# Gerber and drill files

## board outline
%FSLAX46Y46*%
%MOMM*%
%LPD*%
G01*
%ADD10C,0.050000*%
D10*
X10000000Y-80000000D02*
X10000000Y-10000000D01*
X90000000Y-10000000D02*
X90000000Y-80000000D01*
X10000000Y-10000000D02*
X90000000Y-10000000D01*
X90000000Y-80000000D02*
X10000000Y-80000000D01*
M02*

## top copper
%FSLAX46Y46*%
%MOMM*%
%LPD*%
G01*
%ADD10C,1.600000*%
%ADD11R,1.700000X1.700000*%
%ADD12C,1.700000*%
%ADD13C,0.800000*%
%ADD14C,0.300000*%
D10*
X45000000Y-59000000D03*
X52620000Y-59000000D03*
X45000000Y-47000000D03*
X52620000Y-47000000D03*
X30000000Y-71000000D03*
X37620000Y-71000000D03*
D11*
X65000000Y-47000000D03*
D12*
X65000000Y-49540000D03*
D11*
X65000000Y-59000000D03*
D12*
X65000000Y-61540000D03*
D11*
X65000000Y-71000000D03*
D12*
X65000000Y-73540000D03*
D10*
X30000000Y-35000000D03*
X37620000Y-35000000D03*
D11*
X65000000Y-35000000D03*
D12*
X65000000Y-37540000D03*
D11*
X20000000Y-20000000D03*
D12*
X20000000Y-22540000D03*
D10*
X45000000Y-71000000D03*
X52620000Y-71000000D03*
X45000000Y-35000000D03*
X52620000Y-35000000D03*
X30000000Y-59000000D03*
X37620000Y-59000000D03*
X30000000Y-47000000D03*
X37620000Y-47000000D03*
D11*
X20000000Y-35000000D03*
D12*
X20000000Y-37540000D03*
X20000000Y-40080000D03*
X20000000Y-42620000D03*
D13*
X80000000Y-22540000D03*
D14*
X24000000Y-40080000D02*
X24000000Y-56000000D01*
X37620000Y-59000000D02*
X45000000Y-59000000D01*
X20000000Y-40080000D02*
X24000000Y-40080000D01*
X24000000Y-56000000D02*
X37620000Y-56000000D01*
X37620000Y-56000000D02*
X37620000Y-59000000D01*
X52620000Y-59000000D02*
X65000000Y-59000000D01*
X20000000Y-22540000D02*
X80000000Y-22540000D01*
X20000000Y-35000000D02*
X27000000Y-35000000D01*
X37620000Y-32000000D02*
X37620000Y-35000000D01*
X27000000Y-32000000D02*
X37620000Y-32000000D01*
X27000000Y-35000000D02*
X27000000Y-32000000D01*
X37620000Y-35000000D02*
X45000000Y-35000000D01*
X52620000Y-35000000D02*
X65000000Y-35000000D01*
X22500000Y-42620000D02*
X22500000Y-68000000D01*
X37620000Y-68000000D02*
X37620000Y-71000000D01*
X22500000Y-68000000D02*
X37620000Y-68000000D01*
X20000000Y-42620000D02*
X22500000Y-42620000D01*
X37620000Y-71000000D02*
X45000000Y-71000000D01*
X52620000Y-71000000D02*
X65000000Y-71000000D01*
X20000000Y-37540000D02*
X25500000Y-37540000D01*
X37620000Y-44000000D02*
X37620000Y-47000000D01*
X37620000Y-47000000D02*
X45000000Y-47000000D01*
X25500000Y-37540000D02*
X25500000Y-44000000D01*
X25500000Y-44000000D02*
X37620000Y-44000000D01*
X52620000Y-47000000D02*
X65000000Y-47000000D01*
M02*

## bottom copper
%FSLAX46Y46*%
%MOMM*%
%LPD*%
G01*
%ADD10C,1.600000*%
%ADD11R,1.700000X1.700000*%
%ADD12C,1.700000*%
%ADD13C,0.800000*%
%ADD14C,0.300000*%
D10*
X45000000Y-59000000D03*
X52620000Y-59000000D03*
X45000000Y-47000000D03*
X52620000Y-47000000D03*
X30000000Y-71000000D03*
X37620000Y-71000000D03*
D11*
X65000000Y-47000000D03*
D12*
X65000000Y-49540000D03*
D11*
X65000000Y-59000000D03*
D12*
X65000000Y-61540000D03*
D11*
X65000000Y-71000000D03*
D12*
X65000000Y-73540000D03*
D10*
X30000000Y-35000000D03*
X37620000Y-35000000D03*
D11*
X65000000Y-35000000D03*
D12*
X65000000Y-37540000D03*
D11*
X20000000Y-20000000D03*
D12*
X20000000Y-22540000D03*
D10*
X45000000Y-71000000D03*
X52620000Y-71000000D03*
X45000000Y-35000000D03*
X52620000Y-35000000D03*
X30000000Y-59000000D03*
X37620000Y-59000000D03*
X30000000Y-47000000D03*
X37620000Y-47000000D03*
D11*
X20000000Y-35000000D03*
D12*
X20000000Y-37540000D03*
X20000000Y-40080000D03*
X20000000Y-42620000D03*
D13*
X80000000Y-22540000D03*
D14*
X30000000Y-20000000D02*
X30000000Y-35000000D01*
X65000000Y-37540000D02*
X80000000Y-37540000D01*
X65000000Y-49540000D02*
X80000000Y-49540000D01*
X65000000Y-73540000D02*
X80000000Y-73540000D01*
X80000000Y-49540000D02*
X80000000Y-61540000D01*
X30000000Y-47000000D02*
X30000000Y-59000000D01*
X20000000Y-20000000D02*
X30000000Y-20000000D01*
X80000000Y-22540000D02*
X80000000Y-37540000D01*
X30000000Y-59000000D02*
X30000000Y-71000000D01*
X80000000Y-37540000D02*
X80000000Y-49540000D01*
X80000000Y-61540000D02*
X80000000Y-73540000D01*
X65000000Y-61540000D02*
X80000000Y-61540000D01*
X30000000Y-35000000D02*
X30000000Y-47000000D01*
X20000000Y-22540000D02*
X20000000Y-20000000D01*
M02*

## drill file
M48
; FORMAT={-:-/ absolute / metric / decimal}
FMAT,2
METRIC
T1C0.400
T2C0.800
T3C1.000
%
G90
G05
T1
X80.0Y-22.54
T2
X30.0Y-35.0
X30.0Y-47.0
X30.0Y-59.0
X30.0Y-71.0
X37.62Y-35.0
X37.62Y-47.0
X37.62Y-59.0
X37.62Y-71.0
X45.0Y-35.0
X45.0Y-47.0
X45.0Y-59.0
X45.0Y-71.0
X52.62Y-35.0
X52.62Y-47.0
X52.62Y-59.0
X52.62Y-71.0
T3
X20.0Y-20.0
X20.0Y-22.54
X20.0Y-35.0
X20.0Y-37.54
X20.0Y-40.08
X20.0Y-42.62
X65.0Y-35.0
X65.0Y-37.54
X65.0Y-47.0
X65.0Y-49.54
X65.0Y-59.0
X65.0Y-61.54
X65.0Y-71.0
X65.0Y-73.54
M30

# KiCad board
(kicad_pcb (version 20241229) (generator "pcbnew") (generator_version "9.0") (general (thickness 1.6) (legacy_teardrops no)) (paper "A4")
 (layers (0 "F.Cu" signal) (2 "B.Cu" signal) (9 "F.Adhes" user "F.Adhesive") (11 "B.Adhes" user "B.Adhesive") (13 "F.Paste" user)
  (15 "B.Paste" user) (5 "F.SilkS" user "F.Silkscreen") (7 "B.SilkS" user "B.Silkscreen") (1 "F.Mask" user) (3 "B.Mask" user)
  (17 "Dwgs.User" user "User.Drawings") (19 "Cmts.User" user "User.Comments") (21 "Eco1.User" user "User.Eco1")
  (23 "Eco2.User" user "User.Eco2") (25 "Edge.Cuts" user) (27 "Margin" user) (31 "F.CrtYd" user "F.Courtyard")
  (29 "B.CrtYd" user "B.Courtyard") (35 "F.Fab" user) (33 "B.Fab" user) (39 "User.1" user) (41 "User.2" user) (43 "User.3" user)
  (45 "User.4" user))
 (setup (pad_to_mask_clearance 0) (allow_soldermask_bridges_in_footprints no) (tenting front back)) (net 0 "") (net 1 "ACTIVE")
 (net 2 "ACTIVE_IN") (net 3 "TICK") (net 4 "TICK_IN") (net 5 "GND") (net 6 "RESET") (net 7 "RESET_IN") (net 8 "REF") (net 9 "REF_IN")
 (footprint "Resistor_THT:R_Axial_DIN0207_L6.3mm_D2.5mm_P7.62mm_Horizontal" (layer "F.Cu") (at 45 59)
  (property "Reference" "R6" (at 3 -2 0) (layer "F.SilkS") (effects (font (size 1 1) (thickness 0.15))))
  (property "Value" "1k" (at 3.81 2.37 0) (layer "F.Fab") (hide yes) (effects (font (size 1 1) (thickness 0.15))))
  (pad "1" thru_hole circle (at 0 0) (size 1.6 1.6) (drill 0.8) (layers "*.Cu" "*.Mask") (remove_unused_layers no) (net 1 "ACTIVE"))
  (pad "2" thru_hole circle (at 7.62 0) (size 1.6 1.6) (drill 0.8) (layers "*.Cu" "*.Mask") (remove_unused_layers no) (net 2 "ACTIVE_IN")))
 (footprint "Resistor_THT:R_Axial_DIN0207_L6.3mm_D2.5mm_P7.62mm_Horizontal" (layer "F.Cu") (at 45 47)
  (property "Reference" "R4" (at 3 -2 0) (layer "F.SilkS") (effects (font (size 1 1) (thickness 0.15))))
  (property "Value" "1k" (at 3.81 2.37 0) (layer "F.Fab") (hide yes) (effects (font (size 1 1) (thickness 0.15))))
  (pad "1" thru_hole circle (at 0 0) (size 1.6 1.6) (drill 0.8) (layers "*.Cu" "*.Mask") (remove_unused_layers no) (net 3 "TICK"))
  (pad "2" thru_hole circle (at 7.62 0) (size 1.6 1.6) (drill 0.8) (layers "*.Cu" "*.Mask") (remove_unused_layers no) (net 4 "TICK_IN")))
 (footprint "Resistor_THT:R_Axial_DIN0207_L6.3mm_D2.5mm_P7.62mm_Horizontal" (layer "F.Cu") (at 30 71)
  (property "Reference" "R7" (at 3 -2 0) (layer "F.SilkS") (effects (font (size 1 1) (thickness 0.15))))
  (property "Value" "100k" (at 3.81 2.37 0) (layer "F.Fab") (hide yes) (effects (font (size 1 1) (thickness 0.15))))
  (pad "1" thru_hole circle (at 0 0) (size 1.6 1.6) (drill 0.8) (layers "*.Cu" "*.Mask") (remove_unused_layers no) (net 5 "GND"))
  (pad "2" thru_hole circle (at 7.62 0) (size 1.6 1.6) (drill 0.8) (layers "*.Cu" "*.Mask") (remove_unused_layers no) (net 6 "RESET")))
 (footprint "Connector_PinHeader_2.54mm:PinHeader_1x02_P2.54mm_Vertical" (layer "F.Cu") (at 65 47)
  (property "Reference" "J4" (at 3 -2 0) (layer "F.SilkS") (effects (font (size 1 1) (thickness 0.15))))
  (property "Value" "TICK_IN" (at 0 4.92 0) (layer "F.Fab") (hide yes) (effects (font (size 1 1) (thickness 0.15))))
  (pad "1" thru_hole rect (at 0 0) (size 1.7 1.7) (drill 1) (layers "*.Cu" "*.Mask") (remove_unused_layers no) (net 4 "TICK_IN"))
  (pad "2" thru_hole circle (at 0 2.54) (size 1.7 1.7) (drill 1) (layers "*.Cu" "*.Mask") (remove_unused_layers no) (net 5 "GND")))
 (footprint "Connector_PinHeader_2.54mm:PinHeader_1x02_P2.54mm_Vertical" (layer "F.Cu") (at 65 59)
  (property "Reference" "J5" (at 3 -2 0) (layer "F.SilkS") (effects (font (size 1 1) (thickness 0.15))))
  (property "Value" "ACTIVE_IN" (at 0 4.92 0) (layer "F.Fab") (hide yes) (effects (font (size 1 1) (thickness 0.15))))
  (pad "1" thru_hole rect (at 0 0) (size 1.7 1.7) (drill 1) (layers "*.Cu" "*.Mask") (remove_unused_layers no) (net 2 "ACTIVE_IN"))
  (pad "2" thru_hole circle (at 0 2.54) (size 1.7 1.7) (drill 1) (layers "*.Cu" "*.Mask") (remove_unused_layers no) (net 5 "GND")))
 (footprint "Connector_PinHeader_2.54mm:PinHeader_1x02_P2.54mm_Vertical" (layer "F.Cu") (at 65 71)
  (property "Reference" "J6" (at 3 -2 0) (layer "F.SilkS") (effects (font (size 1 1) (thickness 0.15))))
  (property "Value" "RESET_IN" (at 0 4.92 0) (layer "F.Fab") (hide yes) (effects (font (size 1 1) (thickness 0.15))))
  (pad "1" thru_hole rect (at 0 0) (size 1.7 1.7) (drill 1) (layers "*.Cu" "*.Mask") (remove_unused_layers no) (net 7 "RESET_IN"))
  (pad "2" thru_hole circle (at 0 2.54) (size 1.7 1.7) (drill 1) (layers "*.Cu" "*.Mask") (remove_unused_layers no) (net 5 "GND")))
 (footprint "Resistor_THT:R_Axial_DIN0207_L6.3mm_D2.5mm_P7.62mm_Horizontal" (layer "F.Cu") (at 30 35)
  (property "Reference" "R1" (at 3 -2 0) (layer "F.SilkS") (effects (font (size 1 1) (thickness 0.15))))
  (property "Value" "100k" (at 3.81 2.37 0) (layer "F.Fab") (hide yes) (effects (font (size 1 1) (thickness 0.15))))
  (pad "1" thru_hole circle (at 0 0) (size 1.6 1.6) (drill 0.8) (layers "*.Cu" "*.Mask") (remove_unused_layers no) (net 5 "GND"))
  (pad "2" thru_hole circle (at 7.62 0) (size 1.6 1.6) (drill 0.8) (layers "*.Cu" "*.Mask") (remove_unused_layers no) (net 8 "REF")))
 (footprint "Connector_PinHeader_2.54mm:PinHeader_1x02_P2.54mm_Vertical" (layer "F.Cu") (at 65 35)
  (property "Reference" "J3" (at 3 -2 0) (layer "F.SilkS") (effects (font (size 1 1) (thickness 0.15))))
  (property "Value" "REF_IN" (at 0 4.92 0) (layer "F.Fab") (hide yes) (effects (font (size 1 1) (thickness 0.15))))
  (pad "1" thru_hole rect (at 0 0) (size 1.7 1.7) (drill 1) (layers "*.Cu" "*.Mask") (remove_unused_layers no) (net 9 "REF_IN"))
  (pad "2" thru_hole circle (at 0 2.54) (size 1.7 1.7) (drill 1) (layers "*.Cu" "*.Mask") (remove_unused_layers no) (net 5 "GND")))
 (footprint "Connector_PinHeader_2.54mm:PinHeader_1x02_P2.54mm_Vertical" (layer "F.Cu") (at 20 20)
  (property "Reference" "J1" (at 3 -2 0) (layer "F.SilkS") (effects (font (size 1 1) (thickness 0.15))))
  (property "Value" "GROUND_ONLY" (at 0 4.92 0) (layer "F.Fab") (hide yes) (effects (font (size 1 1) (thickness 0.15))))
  (pad "1" thru_hole rect (at 0 0) (size 1.7 1.7) (drill 1) (layers "*.Cu" "*.Mask") (remove_unused_layers no) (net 5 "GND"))
  (pad "2" thru_hole circle (at 0 2.54) (size 1.7 1.7) (drill 1) (layers "*.Cu" "*.Mask") (remove_unused_layers no) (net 5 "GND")))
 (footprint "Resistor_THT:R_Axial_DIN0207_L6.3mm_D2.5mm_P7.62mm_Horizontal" (layer "F.Cu") (at 45 71)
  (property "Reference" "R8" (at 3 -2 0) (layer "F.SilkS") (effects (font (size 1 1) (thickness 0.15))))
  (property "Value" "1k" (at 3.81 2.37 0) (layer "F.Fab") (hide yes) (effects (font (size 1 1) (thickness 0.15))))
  (pad "1" thru_hole circle (at 0 0) (size 1.6 1.6) (drill 0.8) (layers "*.Cu" "*.Mask") (remove_unused_layers no) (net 6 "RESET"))
  (pad "2" thru_hole circle (at 7.62 0) (size 1.6 1.6) (drill 0.8) (layers "*.Cu" "*.Mask") (remove_unused_layers no) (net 7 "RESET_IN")))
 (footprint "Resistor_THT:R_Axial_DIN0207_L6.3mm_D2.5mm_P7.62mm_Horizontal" (layer "F.Cu") (at 45 35)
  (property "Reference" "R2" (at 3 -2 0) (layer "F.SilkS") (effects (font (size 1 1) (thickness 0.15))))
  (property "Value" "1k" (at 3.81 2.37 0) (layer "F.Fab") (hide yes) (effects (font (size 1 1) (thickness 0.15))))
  (pad "1" thru_hole circle (at 0 0) (size 1.6 1.6) (drill 0.8) (layers "*.Cu" "*.Mask") (remove_unused_layers no) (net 8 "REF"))
  (pad "2" thru_hole circle (at 7.62 0) (size 1.6 1.6) (drill 0.8) (layers "*.Cu" "*.Mask") (remove_unused_layers no) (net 9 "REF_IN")))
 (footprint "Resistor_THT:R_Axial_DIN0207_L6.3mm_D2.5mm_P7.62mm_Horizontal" (layer "F.Cu") (at 30 59)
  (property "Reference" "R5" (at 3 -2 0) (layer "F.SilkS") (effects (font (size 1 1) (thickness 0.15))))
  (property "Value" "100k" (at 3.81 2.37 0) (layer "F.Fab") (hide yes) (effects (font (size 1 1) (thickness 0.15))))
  (pad "1" thru_hole circle (at 0 0) (size 1.6 1.6) (drill 0.8) (layers "*.Cu" "*.Mask") (remove_unused_layers no) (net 5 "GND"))
  (pad "2" thru_hole circle (at 7.62 0) (size 1.6 1.6) (drill 0.8) (layers "*.Cu" "*.Mask") (remove_unused_layers no) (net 1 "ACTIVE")))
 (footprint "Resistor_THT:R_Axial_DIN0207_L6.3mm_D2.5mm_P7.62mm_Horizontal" (layer "F.Cu") (at 30 47)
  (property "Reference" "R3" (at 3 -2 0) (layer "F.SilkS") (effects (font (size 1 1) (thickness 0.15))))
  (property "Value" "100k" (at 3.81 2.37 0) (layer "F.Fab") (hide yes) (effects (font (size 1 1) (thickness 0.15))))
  (pad "1" thru_hole circle (at 0 0) (size 1.6 1.6) (drill 0.8) (layers "*.Cu" "*.Mask") (remove_unused_layers no) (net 5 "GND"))
  (pad "2" thru_hole circle (at 7.62 0) (size 1.6 1.6) (drill 0.8) (layers "*.Cu" "*.Mask") (remove_unused_layers no) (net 3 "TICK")))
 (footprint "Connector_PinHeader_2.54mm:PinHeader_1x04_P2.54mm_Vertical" (layer "F.Cu") (at 20 35)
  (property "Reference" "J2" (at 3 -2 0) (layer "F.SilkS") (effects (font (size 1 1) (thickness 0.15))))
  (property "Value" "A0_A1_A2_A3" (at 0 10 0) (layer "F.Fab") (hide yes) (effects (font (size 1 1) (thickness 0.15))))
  (pad "1" thru_hole rect (at 0 0) (size 1.7 1.7) (drill 1) (layers "*.Cu" "*.Mask") (remove_unused_layers no) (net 8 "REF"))
  (pad "2" thru_hole circle (at 0 2.54) (size 1.7 1.7) (drill 1) (layers "*.Cu" "*.Mask") (remove_unused_layers no) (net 3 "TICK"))
  (pad "3" thru_hole circle (at 0 5.08) (size 1.7 1.7) (drill 1) (layers "*.Cu" "*.Mask") (remove_unused_layers no) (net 1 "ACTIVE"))
  (pad "4" thru_hole circle (at 0 7.62) (size 1.7 1.7) (drill 1) (layers "*.Cu" "*.Mask") (remove_unused_layers no) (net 6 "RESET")))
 (gr_line (start 10 80) (end 10 10) (stroke (width 0.05) (type default)) (layer "Edge.Cuts"))
 (gr_line (start 90 10) (end 90 80) (stroke (width 0.05) (type default)) (layer "Edge.Cuts"))
 (gr_line (start 10 10) (end 90 10) (stroke (width 0.05) (type default)) (layer "Edge.Cuts"))
 (gr_line (start 90 80) (end 10 80) (stroke (width 0.05) (type default)) (layer "Edge.Cuts"))
 (segment (start 24 40.08) (end 24 56) (width 0.3) (layer "F.Cu") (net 1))
 (segment (start 37.62 59) (end 45 59) (width 0.3) (layer "F.Cu") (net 1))
 (segment (start 20 40.08) (end 24 40.08) (width 0.3) (layer "F.Cu") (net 1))
 (segment (start 24 56) (end 37.62 56) (width 0.3) (layer "F.Cu") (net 1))
 (segment (start 37.62 56) (end 37.62 59) (width 0.3) (layer "F.Cu") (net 1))
 (segment (start 52.62 59) (end 65 59) (width 0.3) (layer "F.Cu") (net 2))
 (segment (start 20 22.54) (end 80 22.54) (width 0.3) (layer "F.Cu") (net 5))
 (via (at 80 22.54) (size 0.8) (drill 0.4) (layers "F.Cu" "B.Cu") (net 5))
 (segment (start 30 20) (end 30 35) (width 0.3) (layer "B.Cu") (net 5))
 (segment (start 65 37.54) (end 80 37.54) (width 0.3) (layer "B.Cu") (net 5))
 (segment (start 65 49.54) (end 80 49.54) (width 0.3) (layer "B.Cu") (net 5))
 (segment (start 65 73.54) (end 80 73.54) (width 0.3) (layer "B.Cu") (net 5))
 (segment (start 80 49.54) (end 80 61.54) (width 0.3) (layer "B.Cu") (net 5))
 (segment (start 30 47) (end 30 59) (width 0.3) (layer "B.Cu") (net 5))
 (segment (start 20 20) (end 30 20) (width 0.3) (layer "B.Cu") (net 5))
 (segment (start 80 22.54) (end 80 37.54) (width 0.3) (layer "B.Cu") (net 5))
 (segment (start 30 59) (end 30 71) (width 0.3) (layer "B.Cu") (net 5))
 (segment (start 80 37.54) (end 80 49.54) (width 0.3) (layer "B.Cu") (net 5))
 (segment (start 80 61.54) (end 80 73.54) (width 0.3) (layer "B.Cu") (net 5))
 (segment (start 65 61.54) (end 80 61.54) (width 0.3) (layer "B.Cu") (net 5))
 (segment (start 30 35) (end 30 47) (width 0.3) (layer "B.Cu") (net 5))
 (segment (start 20 22.54) (end 20 20) (width 0.3) (layer "B.Cu") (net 5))
 (segment (start 20 35) (end 27 35) (width 0.3) (layer "F.Cu") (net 8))
 (segment (start 37.62 32) (end 37.62 35) (width 0.3) (layer "F.Cu") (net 8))
 (segment (start 27 32) (end 37.62 32) (width 0.3) (layer "F.Cu") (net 8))
 (segment (start 27 35) (end 27 32) (width 0.3) (layer "F.Cu") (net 8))
 (segment (start 37.62 35) (end 45 35) (width 0.3) (layer "F.Cu") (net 8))
 (segment (start 52.62 35) (end 65 35) (width 0.3) (layer "F.Cu") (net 9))
 (segment (start 22.5 42.62) (end 22.5 68) (width 0.3) (layer "F.Cu") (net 6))
 (segment (start 37.62 68) (end 37.62 71) (width 0.3) (layer "F.Cu") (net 6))
 (segment (start 22.5 68) (end 37.62 68) (width 0.3) (layer "F.Cu") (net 6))
 (segment (start 20 42.62) (end 22.5 42.62) (width 0.3) (layer "F.Cu") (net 6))
 (segment (start 37.62 71) (end 45 71) (width 0.3) (layer "F.Cu") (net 6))
 (segment (start 52.62 71) (end 65 71) (width 0.3) (layer "F.Cu") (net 7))
 (segment (start 20 37.54) (end 25.5 37.54) (width 0.3) (layer "F.Cu") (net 3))
 (segment (start 37.62 44) (end 37.62 47) (width 0.3) (layer "F.Cu") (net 3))
 (segment (start 37.62 47) (end 45 47) (width 0.3) (layer "F.Cu") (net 3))
 (segment (start 25.5 37.54) (end 25.5 44) (width 0.3) (layer "F.Cu") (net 3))
 (segment (start 25.5 44) (end 37.62 44) (width 0.3) (layer "F.Cu") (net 3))
 (segment (start 52.62 47) (end 65 47) (width 0.3) (layer "F.Cu") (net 4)))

